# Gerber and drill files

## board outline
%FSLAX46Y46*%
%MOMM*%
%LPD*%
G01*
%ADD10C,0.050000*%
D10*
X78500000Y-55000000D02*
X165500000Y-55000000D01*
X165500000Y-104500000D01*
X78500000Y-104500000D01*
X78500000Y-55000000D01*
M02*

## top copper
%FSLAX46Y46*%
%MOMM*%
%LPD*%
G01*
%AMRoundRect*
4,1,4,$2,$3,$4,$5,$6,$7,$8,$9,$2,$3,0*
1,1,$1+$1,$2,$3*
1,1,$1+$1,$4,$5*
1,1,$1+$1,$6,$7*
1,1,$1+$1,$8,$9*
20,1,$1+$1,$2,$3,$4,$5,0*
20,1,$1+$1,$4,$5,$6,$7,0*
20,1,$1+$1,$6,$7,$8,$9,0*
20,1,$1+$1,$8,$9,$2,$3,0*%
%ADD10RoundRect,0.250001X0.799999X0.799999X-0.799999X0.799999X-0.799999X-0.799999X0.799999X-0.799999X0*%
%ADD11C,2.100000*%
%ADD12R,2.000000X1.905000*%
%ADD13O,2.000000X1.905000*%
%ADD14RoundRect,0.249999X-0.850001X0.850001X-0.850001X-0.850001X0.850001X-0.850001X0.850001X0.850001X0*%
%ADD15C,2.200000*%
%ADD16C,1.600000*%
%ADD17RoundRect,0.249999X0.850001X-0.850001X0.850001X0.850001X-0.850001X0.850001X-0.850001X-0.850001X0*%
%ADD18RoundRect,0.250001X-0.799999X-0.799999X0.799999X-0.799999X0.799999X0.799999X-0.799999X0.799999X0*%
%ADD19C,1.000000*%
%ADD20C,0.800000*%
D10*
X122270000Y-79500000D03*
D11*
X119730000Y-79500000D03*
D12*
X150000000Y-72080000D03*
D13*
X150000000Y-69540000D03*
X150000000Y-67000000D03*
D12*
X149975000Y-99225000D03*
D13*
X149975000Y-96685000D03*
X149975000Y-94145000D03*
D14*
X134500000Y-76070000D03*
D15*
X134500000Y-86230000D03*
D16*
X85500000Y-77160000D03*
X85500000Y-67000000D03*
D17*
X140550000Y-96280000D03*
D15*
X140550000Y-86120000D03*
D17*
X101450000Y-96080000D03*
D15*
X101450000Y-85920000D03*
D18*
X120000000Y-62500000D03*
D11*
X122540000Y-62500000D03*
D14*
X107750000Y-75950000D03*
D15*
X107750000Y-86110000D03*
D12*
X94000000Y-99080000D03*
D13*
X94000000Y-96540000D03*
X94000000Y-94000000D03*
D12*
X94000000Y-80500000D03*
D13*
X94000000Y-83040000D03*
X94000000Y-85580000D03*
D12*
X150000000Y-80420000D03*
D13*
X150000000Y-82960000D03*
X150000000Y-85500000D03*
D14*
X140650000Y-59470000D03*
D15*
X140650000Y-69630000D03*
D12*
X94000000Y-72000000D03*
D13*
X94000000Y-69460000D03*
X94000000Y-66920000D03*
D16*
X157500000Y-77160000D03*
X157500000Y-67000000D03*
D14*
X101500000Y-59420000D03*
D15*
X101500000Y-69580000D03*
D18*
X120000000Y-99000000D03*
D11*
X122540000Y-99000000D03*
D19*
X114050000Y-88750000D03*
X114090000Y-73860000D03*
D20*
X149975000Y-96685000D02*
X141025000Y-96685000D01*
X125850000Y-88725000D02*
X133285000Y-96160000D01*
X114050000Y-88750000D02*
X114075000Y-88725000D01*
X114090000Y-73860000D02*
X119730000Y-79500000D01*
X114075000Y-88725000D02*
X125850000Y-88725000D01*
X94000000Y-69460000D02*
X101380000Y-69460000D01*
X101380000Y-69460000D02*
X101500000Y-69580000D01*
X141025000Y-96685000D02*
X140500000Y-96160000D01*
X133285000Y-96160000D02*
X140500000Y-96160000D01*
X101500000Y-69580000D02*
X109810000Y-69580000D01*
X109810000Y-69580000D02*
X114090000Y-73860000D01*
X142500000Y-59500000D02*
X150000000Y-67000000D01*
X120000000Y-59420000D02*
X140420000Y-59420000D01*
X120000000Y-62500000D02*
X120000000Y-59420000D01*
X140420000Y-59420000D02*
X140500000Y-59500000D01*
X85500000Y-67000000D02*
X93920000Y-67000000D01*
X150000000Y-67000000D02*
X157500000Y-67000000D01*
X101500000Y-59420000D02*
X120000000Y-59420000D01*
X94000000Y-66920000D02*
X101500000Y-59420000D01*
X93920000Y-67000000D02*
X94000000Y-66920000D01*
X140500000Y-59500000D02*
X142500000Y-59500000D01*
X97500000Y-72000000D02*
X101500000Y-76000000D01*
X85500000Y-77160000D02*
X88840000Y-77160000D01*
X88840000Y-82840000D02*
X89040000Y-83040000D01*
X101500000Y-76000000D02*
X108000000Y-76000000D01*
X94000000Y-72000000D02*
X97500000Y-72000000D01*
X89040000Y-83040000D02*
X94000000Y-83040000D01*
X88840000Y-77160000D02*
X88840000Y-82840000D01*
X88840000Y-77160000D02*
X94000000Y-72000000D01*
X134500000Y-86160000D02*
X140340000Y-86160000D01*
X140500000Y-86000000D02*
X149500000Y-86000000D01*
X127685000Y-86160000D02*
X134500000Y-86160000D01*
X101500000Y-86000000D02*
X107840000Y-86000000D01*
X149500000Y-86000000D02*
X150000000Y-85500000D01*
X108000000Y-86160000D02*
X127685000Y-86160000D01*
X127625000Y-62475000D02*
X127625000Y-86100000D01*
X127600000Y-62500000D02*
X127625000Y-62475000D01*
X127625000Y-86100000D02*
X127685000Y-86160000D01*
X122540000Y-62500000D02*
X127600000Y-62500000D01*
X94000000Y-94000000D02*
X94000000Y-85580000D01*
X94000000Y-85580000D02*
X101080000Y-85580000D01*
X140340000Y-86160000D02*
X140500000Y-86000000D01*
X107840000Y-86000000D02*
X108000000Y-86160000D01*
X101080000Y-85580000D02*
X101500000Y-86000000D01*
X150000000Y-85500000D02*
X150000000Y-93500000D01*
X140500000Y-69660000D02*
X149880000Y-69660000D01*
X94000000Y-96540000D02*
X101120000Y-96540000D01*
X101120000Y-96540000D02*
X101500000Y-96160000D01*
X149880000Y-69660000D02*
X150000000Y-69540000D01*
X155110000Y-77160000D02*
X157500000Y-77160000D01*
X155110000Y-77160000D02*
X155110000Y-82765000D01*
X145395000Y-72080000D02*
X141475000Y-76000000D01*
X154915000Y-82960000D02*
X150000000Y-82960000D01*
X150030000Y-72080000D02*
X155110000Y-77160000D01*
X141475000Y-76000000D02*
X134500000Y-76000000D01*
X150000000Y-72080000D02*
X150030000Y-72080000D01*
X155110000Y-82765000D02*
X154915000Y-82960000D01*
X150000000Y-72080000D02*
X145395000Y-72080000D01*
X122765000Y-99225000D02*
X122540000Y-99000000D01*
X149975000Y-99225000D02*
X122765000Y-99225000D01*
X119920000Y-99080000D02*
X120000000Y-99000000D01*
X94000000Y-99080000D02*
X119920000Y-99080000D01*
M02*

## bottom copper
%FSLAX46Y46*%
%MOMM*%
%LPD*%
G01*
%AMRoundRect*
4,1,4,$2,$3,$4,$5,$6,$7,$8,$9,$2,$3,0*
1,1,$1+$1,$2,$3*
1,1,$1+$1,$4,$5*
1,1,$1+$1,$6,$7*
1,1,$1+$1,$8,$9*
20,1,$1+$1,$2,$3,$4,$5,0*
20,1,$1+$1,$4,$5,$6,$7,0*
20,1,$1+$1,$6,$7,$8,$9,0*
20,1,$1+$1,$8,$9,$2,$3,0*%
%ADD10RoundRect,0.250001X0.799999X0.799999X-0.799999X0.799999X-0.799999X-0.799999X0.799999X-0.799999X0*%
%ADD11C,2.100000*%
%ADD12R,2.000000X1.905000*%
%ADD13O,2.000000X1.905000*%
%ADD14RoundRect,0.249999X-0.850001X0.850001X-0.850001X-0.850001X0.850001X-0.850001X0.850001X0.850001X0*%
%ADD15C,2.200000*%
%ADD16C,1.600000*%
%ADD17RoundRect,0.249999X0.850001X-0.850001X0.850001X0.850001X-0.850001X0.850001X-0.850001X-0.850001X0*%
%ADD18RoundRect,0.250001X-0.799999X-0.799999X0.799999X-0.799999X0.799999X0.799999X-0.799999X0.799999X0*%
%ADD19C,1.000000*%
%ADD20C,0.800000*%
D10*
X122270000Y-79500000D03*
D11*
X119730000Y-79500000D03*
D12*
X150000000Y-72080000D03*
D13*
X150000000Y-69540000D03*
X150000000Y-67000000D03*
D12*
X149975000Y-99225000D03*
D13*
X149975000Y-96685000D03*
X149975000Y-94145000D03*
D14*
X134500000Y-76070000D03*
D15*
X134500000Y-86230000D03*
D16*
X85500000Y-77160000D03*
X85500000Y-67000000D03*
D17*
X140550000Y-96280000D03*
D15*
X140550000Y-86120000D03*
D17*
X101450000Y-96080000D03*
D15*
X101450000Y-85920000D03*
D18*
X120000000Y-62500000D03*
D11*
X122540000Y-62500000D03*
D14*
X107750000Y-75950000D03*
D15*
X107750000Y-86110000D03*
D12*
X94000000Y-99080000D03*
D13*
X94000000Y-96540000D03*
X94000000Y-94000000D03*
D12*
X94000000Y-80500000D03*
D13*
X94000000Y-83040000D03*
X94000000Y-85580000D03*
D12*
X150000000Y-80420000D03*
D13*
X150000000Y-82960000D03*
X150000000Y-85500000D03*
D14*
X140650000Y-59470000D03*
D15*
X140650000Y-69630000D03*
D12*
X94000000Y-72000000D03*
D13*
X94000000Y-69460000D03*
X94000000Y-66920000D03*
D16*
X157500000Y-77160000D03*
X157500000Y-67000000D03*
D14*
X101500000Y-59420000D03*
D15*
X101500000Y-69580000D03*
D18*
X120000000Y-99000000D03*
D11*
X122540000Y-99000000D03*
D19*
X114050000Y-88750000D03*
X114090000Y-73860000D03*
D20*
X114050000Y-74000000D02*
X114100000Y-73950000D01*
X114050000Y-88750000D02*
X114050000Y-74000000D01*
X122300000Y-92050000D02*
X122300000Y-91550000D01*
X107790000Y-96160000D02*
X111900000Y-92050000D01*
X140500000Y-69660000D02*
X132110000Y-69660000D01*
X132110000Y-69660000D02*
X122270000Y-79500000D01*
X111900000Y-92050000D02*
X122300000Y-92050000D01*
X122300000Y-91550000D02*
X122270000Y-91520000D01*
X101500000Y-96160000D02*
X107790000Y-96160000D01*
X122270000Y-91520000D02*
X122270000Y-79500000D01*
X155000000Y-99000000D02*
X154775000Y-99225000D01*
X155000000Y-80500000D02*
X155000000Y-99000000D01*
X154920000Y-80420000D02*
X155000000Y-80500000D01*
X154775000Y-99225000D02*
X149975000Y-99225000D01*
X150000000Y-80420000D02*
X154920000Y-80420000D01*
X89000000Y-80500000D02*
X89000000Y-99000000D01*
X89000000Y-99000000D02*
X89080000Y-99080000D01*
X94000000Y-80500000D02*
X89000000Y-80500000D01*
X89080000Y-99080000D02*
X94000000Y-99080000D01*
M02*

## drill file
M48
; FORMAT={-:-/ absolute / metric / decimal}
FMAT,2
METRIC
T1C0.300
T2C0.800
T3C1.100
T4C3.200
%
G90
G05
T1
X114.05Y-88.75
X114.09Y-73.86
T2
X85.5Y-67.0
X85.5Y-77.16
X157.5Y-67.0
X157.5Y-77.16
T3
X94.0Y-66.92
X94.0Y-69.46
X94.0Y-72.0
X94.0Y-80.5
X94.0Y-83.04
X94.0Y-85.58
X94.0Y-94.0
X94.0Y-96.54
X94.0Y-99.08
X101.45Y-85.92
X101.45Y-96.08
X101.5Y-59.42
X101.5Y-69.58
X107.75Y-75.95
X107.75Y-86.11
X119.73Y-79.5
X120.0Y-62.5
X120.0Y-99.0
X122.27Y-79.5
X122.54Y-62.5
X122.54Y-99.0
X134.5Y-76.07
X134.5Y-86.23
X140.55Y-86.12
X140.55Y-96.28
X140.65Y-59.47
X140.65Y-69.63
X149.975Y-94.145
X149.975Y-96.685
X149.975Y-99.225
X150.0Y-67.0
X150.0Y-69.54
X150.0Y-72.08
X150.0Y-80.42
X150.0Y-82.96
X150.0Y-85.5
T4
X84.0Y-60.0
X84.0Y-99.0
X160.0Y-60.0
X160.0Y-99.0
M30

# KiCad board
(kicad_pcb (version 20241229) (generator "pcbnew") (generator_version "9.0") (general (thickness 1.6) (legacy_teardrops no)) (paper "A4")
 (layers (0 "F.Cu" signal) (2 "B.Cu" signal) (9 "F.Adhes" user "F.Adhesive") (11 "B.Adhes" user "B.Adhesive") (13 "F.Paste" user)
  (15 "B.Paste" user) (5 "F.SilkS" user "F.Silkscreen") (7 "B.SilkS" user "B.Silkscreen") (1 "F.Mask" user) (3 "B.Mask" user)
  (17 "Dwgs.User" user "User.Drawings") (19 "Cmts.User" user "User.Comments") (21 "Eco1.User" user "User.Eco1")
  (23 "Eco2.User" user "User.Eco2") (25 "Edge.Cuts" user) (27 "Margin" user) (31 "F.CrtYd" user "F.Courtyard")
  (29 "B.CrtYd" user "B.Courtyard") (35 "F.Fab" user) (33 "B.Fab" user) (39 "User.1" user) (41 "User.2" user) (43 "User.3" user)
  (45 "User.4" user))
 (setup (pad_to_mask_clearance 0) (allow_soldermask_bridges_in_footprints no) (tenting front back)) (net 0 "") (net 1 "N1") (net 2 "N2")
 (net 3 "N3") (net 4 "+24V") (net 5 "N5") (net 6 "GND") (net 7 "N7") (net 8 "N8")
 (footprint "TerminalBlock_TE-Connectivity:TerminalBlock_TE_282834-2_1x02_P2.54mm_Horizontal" (layer "F.Cu") (at 122.27 79.5 180)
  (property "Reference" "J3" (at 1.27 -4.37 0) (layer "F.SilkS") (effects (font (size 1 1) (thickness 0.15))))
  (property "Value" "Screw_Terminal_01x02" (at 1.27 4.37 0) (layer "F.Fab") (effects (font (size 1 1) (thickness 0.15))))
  (pad "1" thru_hole roundrect (at 0 0 180) (size 2.1 2.1) (drill 1.1) (layers "*.Cu" "*.Mask") (remove_unused_layers no)
   (roundrect_rratio 0.119048) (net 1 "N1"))
  (pad "2" thru_hole circle (at 2.54 0 180) (size 2.1 2.1) (drill 1.1) (layers "*.Cu" "*.Mask") (remove_unused_layers no) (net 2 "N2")))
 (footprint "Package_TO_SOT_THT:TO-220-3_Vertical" (layer "F.Cu") (at 150 72.08 90)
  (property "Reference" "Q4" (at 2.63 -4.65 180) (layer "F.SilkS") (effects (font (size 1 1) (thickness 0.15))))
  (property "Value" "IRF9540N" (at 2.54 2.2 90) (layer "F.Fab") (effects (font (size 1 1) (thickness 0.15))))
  (pad "1" thru_hole rect (at 0 0 90) (size 1.905 2) (drill 1.1) (layers "*.Cu" "*.Mask") (remove_unused_layers no) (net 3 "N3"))
  (pad "2" thru_hole oval (at 2.54 0 90) (size 1.905 2) (drill 1.1) (layers "*.Cu" "*.Mask") (remove_unused_layers no) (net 1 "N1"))
  (pad "3" thru_hole oval (at 5.08 0 90) (size 1.905 2) (drill 1.1) (layers "*.Cu" "*.Mask") (remove_unused_layers no) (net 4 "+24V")))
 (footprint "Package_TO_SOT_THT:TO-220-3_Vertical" (layer "F.Cu") (at 149.975 99.225 90)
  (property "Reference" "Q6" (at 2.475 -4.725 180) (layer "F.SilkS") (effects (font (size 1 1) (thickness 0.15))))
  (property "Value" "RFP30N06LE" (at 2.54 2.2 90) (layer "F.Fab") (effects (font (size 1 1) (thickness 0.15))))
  (pad "1" thru_hole rect (at 0 0 90) (size 1.905 2) (drill 1.1) (layers "*.Cu" "*.Mask") (remove_unused_layers no) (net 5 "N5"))
  (pad "2" thru_hole oval (at 2.54 0 90) (size 1.905 2) (drill 1.1) (layers "*.Cu" "*.Mask") (remove_unused_layers no) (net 2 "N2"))
  (pad "3" thru_hole oval (at 5.08 0 90) (size 1.905 2) (drill 1.1) (layers "*.Cu" "*.Mask") (remove_unused_layers no) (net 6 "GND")))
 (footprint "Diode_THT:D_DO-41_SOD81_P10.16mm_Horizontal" (layer "F.Cu") (at 134.5 76.07 -90)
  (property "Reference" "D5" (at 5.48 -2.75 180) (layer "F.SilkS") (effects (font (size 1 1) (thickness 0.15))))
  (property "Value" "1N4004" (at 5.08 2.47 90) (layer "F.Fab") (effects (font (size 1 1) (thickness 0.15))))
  (pad "1" thru_hole roundrect (at 0 0 270) (size 2.2 2.2) (drill 1.1) (layers "*.Cu" "*.Mask") (remove_unused_layers no)
   (roundrect_rratio 0.113636) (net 3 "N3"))
  (pad "2" thru_hole circle (at 10.16 0 270) (size 2.2 2.2) (drill 1.1) (layers "*.Cu" "*.Mask") (remove_unused_layers no) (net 6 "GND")))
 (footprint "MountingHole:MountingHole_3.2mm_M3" (layer "F.Cu") (at 84 99)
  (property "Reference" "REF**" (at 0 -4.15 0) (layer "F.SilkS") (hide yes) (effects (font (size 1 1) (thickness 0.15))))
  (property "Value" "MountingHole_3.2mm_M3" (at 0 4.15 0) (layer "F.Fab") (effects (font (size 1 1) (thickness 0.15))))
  (pad "" np_thru_hole circle (at 0 0) (size 3.2 3.2) (drill 3.2) (layers "*.Cu" "*.Mask")))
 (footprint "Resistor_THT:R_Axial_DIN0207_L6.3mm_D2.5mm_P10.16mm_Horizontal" (layer "F.Cu") (at 85.5 77.16 90)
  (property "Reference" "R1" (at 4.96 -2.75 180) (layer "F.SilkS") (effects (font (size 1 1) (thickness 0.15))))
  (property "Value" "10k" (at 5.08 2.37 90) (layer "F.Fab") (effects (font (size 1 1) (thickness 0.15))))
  (pad "1" thru_hole circle (at 0 0 90) (size 1.6 1.6) (drill 0.8) (layers "*.Cu" "*.Mask") (remove_unused_layers no) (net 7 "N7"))
  (pad "2" thru_hole circle (at 10.16 0 90) (size 1.6 1.6) (drill 0.8) (layers "*.Cu" "*.Mask") (remove_unused_layers no) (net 4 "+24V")))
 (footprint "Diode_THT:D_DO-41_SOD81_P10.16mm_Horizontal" (layer "F.Cu") (at 140.55 96.28 90)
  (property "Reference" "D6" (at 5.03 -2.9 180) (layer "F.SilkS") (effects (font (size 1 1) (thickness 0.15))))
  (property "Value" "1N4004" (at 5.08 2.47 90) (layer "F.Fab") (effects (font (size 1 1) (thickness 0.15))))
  (pad "1" thru_hole roundrect (at 0 0 90) (size 2.2 2.2) (drill 1.1) (layers "*.Cu" "*.Mask") (remove_unused_layers no)
   (roundrect_rratio 0.113636) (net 2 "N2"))
  (pad "2" thru_hole circle (at 10.16 0 90) (size 2.2 2.2) (drill 1.1) (layers "*.Cu" "*.Mask") (remove_unused_layers no) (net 6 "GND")))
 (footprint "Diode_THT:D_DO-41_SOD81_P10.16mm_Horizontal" (layer "F.Cu") (at 101.45 96.08 90)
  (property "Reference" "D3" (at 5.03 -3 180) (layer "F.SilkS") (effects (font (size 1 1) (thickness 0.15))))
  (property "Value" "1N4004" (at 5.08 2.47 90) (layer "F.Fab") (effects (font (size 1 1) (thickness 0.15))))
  (pad "1" thru_hole roundrect (at 0 0 90) (size 2.2 2.2) (drill 1.1) (layers "*.Cu" "*.Mask") (remove_unused_layers no)
   (roundrect_rratio 0.113636) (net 1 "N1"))
  (pad "2" thru_hole circle (at 10.16 0 90) (size 2.2 2.2) (drill 1.1) (layers "*.Cu" "*.Mask") (remove_unused_layers no) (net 6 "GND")))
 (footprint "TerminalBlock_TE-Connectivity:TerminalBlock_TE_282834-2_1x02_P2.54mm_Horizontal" (layer "F.Cu") (at 120 62.5)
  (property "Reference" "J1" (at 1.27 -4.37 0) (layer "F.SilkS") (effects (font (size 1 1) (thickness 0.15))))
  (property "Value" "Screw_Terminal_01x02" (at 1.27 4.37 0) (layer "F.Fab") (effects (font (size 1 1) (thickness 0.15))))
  (pad "1" thru_hole roundrect (at 0 0) (size 2.1 2.1) (drill 1.1) (layers "*.Cu" "*.Mask") (remove_unused_layers no)
   (roundrect_rratio 0.119048) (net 4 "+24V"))
  (pad "2" thru_hole circle (at 2.54 0) (size 2.1 2.1) (drill 1.1) (layers "*.Cu" "*.Mask") (remove_unused_layers no) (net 6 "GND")))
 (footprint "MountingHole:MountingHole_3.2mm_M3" (layer "F.Cu") (at 84 60)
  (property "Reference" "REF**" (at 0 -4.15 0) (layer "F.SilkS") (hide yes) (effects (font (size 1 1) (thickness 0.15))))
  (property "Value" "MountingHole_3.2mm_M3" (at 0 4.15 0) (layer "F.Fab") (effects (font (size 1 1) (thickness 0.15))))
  (pad "" np_thru_hole circle (at 0 0) (size 3.2 3.2) (drill 3.2) (layers "*.Cu" "*.Mask")))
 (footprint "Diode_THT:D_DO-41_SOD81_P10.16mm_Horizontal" (layer "F.Cu") (at 107.75 75.95 -90)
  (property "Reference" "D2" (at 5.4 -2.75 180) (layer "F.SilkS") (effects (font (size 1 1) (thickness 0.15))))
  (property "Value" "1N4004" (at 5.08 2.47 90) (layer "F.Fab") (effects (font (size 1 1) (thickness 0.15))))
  (pad "1" thru_hole roundrect (at 0 0 270) (size 2.2 2.2) (drill 1.1) (layers "*.Cu" "*.Mask") (remove_unused_layers no)
   (roundrect_rratio 0.113636) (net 7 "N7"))
  (pad "2" thru_hole circle (at 10.16 0 270) (size 2.2 2.2) (drill 1.1) (layers "*.Cu" "*.Mask") (remove_unused_layers no) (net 6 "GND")))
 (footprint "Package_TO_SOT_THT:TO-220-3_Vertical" (layer "F.Cu") (at 94 99.08 90)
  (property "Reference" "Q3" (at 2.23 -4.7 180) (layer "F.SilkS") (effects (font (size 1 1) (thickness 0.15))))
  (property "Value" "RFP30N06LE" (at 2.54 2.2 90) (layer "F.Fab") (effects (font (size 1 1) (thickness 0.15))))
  (pad "1" thru_hole rect (at 0 0 90) (size 1.905 2) (drill 1.1) (layers "*.Cu" "*.Mask") (remove_unused_layers no) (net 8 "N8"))
  (pad "2" thru_hole oval (at 2.54 0 90) (size 1.905 2) (drill 1.1) (layers "*.Cu" "*.Mask") (remove_unused_layers no) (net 1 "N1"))
  (pad "3" thru_hole oval (at 5.08 0 90) (size 1.905 2) (drill 1.1) (layers "*.Cu" "*.Mask") (remove_unused_layers no) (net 6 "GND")))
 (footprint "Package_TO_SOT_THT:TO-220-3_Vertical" (layer "F.Cu") (at 94 80.5 -90)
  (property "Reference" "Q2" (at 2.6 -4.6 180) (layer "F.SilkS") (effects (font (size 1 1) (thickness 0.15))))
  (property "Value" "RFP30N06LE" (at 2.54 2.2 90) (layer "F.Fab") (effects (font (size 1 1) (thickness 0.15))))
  (pad "1" thru_hole rect (at 0 0 270) (size 1.905 2) (drill 1.1) (layers "*.Cu" "*.Mask") (remove_unused_layers no) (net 8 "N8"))
  (pad "2" thru_hole oval (at 2.54 0 270) (size 1.905 2) (drill 1.1) (layers "*.Cu" "*.Mask") (remove_unused_layers no) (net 7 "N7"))
  (pad "3" thru_hole oval (at 5.08 0 270) (size 1.905 2) (drill 1.1) (layers "*.Cu" "*.Mask") (remove_unused_layers no) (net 6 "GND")))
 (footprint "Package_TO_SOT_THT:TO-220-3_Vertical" (layer "F.Cu") (at 150 80.42 -90)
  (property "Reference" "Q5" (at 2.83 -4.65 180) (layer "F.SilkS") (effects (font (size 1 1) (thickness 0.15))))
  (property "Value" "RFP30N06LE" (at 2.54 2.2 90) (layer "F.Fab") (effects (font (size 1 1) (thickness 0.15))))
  (pad "1" thru_hole rect (at 0 0 270) (size 1.905 2) (drill 1.1) (layers "*.Cu" "*.Mask") (remove_unused_layers no) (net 5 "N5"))
  (pad "2" thru_hole oval (at 2.54 0 270) (size 1.905 2) (drill 1.1) (layers "*.Cu" "*.Mask") (remove_unused_layers no) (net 3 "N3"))
  (pad "3" thru_hole oval (at 5.08 0 270) (size 1.905 2) (drill 1.1) (layers "*.Cu" "*.Mask") (remove_unused_layers no) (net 6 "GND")))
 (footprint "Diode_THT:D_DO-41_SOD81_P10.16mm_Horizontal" (layer "F.Cu") (at 140.65 59.47 -90)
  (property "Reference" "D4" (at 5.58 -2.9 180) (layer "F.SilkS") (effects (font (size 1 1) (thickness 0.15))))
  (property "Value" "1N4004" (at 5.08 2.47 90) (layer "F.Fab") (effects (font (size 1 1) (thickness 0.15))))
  (pad "1" thru_hole roundrect (at 0 0 270) (size 2.2 2.2) (drill 1.1) (layers "*.Cu" "*.Mask") (remove_unused_layers no)
   (roundrect_rratio 0.113636) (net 4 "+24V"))
  (pad "2" thru_hole circle (at 10.16 0 270) (size 2.2 2.2) (drill 1.1) (layers "*.Cu" "*.Mask") (remove_unused_layers no) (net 1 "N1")))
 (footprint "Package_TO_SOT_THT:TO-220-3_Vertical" (layer "F.Cu") (at 94 72 90)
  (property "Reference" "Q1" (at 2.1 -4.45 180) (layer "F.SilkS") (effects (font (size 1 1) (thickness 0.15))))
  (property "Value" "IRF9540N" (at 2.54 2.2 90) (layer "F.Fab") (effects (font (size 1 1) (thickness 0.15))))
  (pad "1" thru_hole rect (at 0 0 90) (size 1.905 2) (drill 1.1) (layers "*.Cu" "*.Mask") (remove_unused_layers no) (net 7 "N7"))
  (pad "2" thru_hole oval (at 2.54 0 90) (size 1.905 2) (drill 1.1) (layers "*.Cu" "*.Mask") (remove_unused_layers no) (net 2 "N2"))
  (pad "3" thru_hole oval (at 5.08 0 90) (size 1.905 2) (drill 1.1) (layers "*.Cu" "*.Mask") (remove_unused_layers no) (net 4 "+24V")))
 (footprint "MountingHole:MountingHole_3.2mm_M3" (layer "F.Cu") (at 160 60)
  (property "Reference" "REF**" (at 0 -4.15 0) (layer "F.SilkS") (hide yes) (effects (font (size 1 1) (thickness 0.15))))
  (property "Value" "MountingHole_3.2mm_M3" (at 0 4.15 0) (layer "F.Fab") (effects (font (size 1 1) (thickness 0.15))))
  (pad "" np_thru_hole circle (at 0 0) (size 3.2 3.2) (drill 3.2) (layers "*.Cu" "*.Mask")))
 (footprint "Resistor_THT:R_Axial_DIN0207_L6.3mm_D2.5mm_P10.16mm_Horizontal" (layer "F.Cu") (at 157.5 77.16 90)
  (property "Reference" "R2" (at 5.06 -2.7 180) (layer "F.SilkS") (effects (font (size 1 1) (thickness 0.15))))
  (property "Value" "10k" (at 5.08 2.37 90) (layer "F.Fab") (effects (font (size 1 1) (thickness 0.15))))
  (pad "1" thru_hole circle (at 0 0 90) (size 1.6 1.6) (drill 0.8) (layers "*.Cu" "*.Mask") (remove_unused_layers no) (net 3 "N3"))
  (pad "2" thru_hole circle (at 10.16 0 90) (size 1.6 1.6) (drill 0.8) (layers "*.Cu" "*.Mask") (remove_unused_layers no) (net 4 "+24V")))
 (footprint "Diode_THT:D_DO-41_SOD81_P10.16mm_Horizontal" (layer "F.Cu") (at 101.5 59.42 -90)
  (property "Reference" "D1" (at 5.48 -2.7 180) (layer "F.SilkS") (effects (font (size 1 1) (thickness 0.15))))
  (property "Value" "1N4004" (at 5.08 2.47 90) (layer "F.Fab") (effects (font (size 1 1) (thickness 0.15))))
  (pad "1" thru_hole roundrect (at 0 0 270) (size 2.2 2.2) (drill 1.1) (layers "*.Cu" "*.Mask") (remove_unused_layers no)
   (roundrect_rratio 0.113636) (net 4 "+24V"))
  (pad "2" thru_hole circle (at 10.16 0 270) (size 2.2 2.2) (drill 1.1) (layers "*.Cu" "*.Mask") (remove_unused_layers no) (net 2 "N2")))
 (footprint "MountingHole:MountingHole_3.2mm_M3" (layer "F.Cu") (at 160 99)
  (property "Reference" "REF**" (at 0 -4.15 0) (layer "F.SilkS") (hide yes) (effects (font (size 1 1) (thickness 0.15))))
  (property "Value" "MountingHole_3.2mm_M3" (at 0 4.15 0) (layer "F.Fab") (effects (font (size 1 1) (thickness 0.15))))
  (pad "" np_thru_hole circle (at 0 0) (size 3.2 3.2) (drill 3.2) (layers "*.Cu" "*.Mask")))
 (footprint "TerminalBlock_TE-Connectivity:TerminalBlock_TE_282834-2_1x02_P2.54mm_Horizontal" (layer "F.Cu") (at 120 99)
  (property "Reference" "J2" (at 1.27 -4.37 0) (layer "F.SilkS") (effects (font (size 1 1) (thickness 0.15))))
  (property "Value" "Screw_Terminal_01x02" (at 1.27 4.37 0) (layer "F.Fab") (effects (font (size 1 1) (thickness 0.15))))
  (pad "1" thru_hole roundrect (at 0 0) (size 2.1 2.1) (drill 1.1) (layers "*.Cu" "*.Mask") (remove_unused_layers no)
   (roundrect_rratio 0.119048) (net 8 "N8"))
  (pad "2" thru_hole circle (at 2.54 0) (size 2.1 2.1) (drill 1.1) (layers "*.Cu" "*.Mask") (remove_unused_layers no) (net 5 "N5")))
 (gr_rect (start 78.5 55) (end 165.5 104.5) (stroke (width 0.05) (type default)) (fill no) (layer "Edge.Cuts"))
 (segment (start 149.975 96.685) (end 141.025 96.685) (width 0.8) (layer "F.Cu") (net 2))
 (segment (start 125.85 88.725) (end 133.285 96.16) (width 0.8) (layer "F.Cu") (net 2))
 (segment (start 114.05 88.75) (end 114.075 88.725) (width 0.8) (layer "F.Cu") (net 2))
 (segment (start 114.09 73.86) (end 119.73 79.5) (width 0.8) (layer "F.Cu") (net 2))
 (segment (start 114.075 88.725) (end 125.85 88.725) (width 0.8) (layer "F.Cu") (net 2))
 (segment (start 94 69.46) (end 101.38 69.46) (width 0.8) (layer "F.Cu") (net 2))
 (segment (start 101.38 69.46) (end 101.5 69.58) (width 0.8) (layer "F.Cu") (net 2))
 (segment (start 141.025 96.685) (end 140.5 96.16) (width 0.8) (layer "F.Cu") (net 2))
 (segment (start 133.285 96.16) (end 140.5 96.16) (width 0.8) (layer "F.Cu") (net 2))
 (segment (start 101.5 69.58) (end 109.81 69.58) (width 0.8) (layer "F.Cu") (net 2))
 (segment (start 109.81 69.58) (end 114.09 73.86) (width 0.8) (layer "F.Cu") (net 2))
 (via (at 114.05 88.75) (size 1) (drill 0.3) (layers "F.Cu" "B.Cu") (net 2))
 (via (at 114.09 73.86) (size 1) (drill 0.3) (layers "F.Cu" "B.Cu") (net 2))
 (segment (start 114.05 74) (end 114.1 73.95) (width 0.8) (layer "B.Cu") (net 2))
 (segment (start 114.05 88.75) (end 114.05 74) (width 0.8) (layer "B.Cu") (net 2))
 (segment (start 142.5 59.5) (end 150 67) (width 0.8) (layer "F.Cu") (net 4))
 (segment (start 120 59.42) (end 140.42 59.42) (width 0.8) (layer "F.Cu") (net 4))
 (segment (start 120 62.5) (end 120 59.42) (width 0.8) (layer "F.Cu") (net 4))
 (segment (start 140.42 59.42) (end 140.5 59.5) (width 0.8) (layer "F.Cu") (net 4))
 (segment (start 85.5 67) (end 93.92 67) (width 0.8) (layer "F.Cu") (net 4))
 (segment (start 150 67) (end 157.5 67) (width 0.8) (layer "F.Cu") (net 4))
 (segment (start 101.5 59.42) (end 120 59.42) (width 0.8) (layer "F.Cu") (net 4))
 (segment (start 94 66.92) (end 101.5 59.42) (width 0.8) (layer "F.Cu") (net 4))
 (segment (start 93.92 67) (end 94 66.92) (width 0.8) (layer "F.Cu") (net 4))
 (segment (start 140.5 59.5) (end 142.5 59.5) (width 0.8) (layer "F.Cu") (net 4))
 (segment (start 97.5 72) (end 101.5 76) (width 0.8) (layer "F.Cu") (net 7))
 (segment (start 85.5 77.16) (end 88.84 77.16) (width 0.8) (layer "F.Cu") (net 7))
 (segment (start 88.84 82.84) (end 89.04 83.04) (width 0.8) (layer "F.Cu") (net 7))
 (segment (start 101.5 76) (end 108 76) (width 0.8) (layer "F.Cu") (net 7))
 (segment (start 94 72) (end 97.5 72) (width 0.8) (layer "F.Cu") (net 7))
 (segment (start 89.04 83.04) (end 94 83.04) (width 0.8) (layer "F.Cu") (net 7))
 (segment (start 88.84 77.16) (end 88.84 82.84) (width 0.8) (layer "F.Cu") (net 7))
 (segment (start 88.84 77.16) (end 94 72) (width 0.8) (layer "F.Cu") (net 7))
 (segment (start 134.5 86.16) (end 140.34 86.16) (width 0.8) (layer "F.Cu") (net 6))
 (segment (start 140.5 86) (end 149.5 86) (width 0.8) (layer "F.Cu") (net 6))
 (segment (start 127.685 86.16) (end 134.5 86.16) (width 0.8) (layer "F.Cu") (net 6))
 (segment (start 101.5 86) (end 107.84 86) (width 0.8) (layer "F.Cu") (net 6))
 (segment (start 149.5 86) (end 150 85.5) (width 0.8) (layer "F.Cu") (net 6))
 (segment (start 108 86.16) (end 127.685 86.16) (width 0.8) (layer "F.Cu") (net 6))
 (segment (start 127.625 62.475) (end 127.625 86.1) (width 0.8) (layer "F.Cu") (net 6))
 (segment (start 127.6 62.5) (end 127.625 62.475) (width 0.8) (layer "F.Cu") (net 6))
 (segment (start 127.625 86.1) (end 127.685 86.16) (width 0.8) (layer "F.Cu") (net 6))
 (segment (start 122.54 62.5) (end 127.6 62.5) (width 0.8) (layer "F.Cu") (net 6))
 (segment (start 94 94) (end 94 85.58) (width 0.8) (layer "F.Cu") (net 6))
 (segment (start 94 85.58) (end 101.08 85.58) (width 0.8) (layer "F.Cu") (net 6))
 (segment (start 140.34 86.16) (end 140.5 86) (width 0.8) (layer "F.Cu") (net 6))
 (segment (start 107.84 86) (end 108 86.16) (width 0.8) (layer "F.Cu") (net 6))
 (segment (start 101.08 85.58) (end 101.5 86) (width 0.8) (layer "F.Cu") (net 6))
 (segment (start 150 85.5) (end 150 93.5) (width 0.8) (layer "F.Cu") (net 6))
 (segment (start 140.5 69.66) (end 149.88 69.66) (width 0.8) (layer "F.Cu") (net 1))
 (segment (start 94 96.54) (end 101.12 96.54) (width 0.8) (layer "F.Cu") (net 1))
 (segment (start 101.12 96.54) (end 101.5 96.16) (width 0.8) (layer "F.Cu") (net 1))
 (segment (start 149.88 69.66) (end 150 69.54) (width 0.8) (layer "F.Cu") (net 1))
 (segment (start 122.3 92.05) (end 122.3 91.55) (width 0.8) (layer "B.Cu") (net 1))
 (segment (start 107.79 96.16) (end 111.9 92.05) (width 0.8) (layer "B.Cu") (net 1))
 (segment (start 140.5 69.66) (end 132.11 69.66) (width 0.8) (layer "B.Cu") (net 1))
 (segment (start 132.11 69.66) (end 122.27 79.5) (width 0.8) (layer "B.Cu") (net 1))
 (segment (start 111.9 92.05) (end 122.3 92.05) (width 0.8) (layer "B.Cu") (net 1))
 (segment (start 122.3 91.55) (end 122.27 91.52) (width 0.8) (layer "B.Cu") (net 1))
 (segment (start 101.5 96.16) (end 107.79 96.16) (width 0.8) (layer "B.Cu") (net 1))
 (segment (start 122.27 91.52) (end 122.27 79.5) (width 0.8) (layer "B.Cu") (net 1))
 (segment (start 155.11 77.16) (end 157.5 77.16) (width 0.8) (layer "F.Cu") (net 3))
 (segment (start 155.11 77.16) (end 155.11 82.765) (width 0.8) (layer "F.Cu") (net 3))
 (segment (start 145.395 72.08) (end 141.475 76) (width 0.8) (layer "F.Cu") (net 3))
 (segment (start 154.915 82.96) (end 150 82.96) (width 0.8) (layer "F.Cu") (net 3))
 (segment (start 150.03 72.08) (end 155.11 77.16) (width 0.8) (layer "F.Cu") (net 3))
 (segment (start 141.475 76) (end 134.5 76) (width 0.8) (layer "F.Cu") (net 3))
 (segment (start 150 72.08) (end 150.03 72.08) (width 0.8) (layer "F.Cu") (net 3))
 (segment (start 155.11 82.765) (end 154.915 82.96) (width 0.8) (layer "F.Cu") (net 3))
 (segment (start 150 72.08) (end 145.395 72.08) (width 0.8) (layer "F.Cu") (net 3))
 (segment (start 122.765 99.225) (end 122.54 99) (width 0.8) (layer "F.Cu") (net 5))
 (segment (start 149.975 99.225) (end 122.765 99.225) (width 0.8) (layer "F.Cu") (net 5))
 (segment (start 155 99) (end 154.775 99.225) (width 0.8) (layer "B.Cu") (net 5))
 (segment (start 155 80.5) (end 155 99) (width 0.8) (layer "B.Cu") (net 5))
 (segment (start 154.92 80.42) (end 155 80.5) (width 0.8) (layer "B.Cu") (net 5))
 (segment (start 154.775 99.225) (end 149.975 99.225) (width 0.8) (layer "B.Cu") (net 5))
 (segment (start 150 80.42) (end 154.92 80.42) (width 0.8) (layer "B.Cu") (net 5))
 (segment (start 119.92 99.08) (end 120 99) (width 0.8) (layer "F.Cu") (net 8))
 (segment (start 94 99.08) (end 119.92 99.08) (width 0.8) (layer "F.Cu") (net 8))
 (segment (start 89 80.5) (end 89 99) (width 0.8) (layer "B.Cu") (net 8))
 (segment (start 89 99) (end 89.08 99.08) (width 0.8) (layer "B.Cu") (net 8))
 (segment (start 94 80.5) (end 89 80.5) (width 0.8) (layer "B.Cu") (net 8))
 (segment (start 89.08 99.08) (end 94 99.08) (width 0.8) (layer "B.Cu") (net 8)))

